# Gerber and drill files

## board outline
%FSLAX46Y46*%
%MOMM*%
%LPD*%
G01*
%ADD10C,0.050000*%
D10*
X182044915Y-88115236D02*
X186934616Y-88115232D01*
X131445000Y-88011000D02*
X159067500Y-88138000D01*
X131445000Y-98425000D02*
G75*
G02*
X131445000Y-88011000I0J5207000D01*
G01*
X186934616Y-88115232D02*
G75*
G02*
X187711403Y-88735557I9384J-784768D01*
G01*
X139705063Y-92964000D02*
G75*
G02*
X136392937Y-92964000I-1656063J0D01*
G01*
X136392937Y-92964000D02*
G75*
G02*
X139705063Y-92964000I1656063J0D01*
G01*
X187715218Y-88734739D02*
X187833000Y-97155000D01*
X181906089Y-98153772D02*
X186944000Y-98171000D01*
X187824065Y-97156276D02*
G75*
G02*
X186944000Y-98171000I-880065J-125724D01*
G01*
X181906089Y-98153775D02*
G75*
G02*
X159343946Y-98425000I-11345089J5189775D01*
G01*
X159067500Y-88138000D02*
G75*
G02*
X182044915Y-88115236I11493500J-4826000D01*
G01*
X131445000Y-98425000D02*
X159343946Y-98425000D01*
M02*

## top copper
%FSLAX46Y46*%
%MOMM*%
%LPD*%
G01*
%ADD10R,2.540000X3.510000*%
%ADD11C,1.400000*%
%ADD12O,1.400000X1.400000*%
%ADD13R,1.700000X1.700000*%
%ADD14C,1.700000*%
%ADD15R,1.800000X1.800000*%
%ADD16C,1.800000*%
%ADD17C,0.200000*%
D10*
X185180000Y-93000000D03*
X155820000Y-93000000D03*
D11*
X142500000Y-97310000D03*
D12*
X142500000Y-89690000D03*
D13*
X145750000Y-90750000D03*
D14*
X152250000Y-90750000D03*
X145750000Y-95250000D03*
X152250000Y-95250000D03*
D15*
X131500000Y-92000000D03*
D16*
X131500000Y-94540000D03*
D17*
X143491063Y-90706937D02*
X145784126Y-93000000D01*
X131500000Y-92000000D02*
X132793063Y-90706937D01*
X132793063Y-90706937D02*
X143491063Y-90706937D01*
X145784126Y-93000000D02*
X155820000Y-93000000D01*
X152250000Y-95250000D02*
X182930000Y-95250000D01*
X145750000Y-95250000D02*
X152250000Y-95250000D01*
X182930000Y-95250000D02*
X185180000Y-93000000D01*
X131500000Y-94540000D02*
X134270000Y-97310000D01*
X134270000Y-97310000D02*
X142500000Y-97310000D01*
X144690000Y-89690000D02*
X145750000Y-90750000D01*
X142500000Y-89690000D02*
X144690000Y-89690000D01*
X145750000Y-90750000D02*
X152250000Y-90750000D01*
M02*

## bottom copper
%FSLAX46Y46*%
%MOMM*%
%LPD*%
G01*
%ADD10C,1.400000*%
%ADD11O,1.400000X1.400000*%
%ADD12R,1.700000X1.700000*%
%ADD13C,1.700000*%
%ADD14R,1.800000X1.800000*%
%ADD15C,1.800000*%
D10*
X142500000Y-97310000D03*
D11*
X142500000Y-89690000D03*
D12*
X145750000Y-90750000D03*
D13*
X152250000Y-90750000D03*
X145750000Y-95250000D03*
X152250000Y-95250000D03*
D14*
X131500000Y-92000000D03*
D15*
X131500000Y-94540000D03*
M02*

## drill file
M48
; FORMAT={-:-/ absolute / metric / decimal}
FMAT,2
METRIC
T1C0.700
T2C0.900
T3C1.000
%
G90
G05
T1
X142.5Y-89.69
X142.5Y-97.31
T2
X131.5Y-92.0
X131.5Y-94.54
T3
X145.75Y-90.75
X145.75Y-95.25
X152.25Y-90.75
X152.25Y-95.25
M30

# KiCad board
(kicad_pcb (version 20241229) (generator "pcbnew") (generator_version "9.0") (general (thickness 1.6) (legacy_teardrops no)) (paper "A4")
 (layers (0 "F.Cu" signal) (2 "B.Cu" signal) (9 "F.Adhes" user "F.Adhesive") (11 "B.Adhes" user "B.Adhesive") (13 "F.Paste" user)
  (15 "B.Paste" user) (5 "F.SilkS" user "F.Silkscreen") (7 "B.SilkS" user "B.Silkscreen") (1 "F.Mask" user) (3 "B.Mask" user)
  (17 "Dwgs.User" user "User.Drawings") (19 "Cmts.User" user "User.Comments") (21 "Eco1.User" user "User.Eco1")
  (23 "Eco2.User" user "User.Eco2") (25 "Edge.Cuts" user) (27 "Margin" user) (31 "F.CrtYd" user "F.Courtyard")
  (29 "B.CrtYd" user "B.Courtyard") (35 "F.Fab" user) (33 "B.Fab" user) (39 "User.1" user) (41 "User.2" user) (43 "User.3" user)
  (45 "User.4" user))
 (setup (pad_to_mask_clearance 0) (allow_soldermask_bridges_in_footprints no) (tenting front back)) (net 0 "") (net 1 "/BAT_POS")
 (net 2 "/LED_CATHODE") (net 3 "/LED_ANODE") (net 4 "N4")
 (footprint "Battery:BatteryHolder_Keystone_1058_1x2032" (layer "F.Cu") (at 170.5 93 180)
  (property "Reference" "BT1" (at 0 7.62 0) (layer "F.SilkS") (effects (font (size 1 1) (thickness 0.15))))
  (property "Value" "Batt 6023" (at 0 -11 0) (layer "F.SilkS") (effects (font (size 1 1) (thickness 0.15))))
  (pad "1" smd rect (at -14.68 0 180) (size 2.54 3.51) (layers "F.Cu" "F.Mask" "F.Paste") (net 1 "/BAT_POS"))
  (pad "2" smd rect (at 14.68 0 180) (size 2.54 3.51) (layers "F.Cu" "F.Mask" "F.Paste") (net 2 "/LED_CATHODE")))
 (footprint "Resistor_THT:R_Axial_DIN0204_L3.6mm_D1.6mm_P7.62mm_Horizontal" (layer "F.Cu") (at 142.5 97.31 90)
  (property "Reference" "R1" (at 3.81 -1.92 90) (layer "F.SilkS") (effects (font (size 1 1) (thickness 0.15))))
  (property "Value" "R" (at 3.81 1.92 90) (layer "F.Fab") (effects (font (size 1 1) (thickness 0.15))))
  (pad "1" thru_hole circle (at 0 0 90) (size 1.4 1.4) (drill 0.7) (layers "*.Cu" "*.Mask") (remove_unused_layers no) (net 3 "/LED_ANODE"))
  (pad "2" thru_hole oval (at 7.62 0 90) (size 1.4 1.4) (drill 0.7) (layers "*.Cu" "*.Mask") (remove_unused_layers no) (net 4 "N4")))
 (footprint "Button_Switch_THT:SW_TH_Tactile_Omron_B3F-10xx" (layer "F.Cu") (at 145.75 90.75)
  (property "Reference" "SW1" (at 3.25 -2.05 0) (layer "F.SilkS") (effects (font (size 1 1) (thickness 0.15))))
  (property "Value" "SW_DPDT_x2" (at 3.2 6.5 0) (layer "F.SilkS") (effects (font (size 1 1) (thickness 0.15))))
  (pad "1" thru_hole rect (at 0 0) (size 1.7 1.7) (drill 1) (layers "*.Cu" "*.Mask") (remove_unused_layers no) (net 4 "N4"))
  (pad "1" thru_hole circle (at 6.5 0) (size 1.7 1.7) (drill 1) (layers "*.Cu" "*.Mask") (remove_unused_layers no) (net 4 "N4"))
  (pad "2" thru_hole circle (at 0 4.5) (size 1.7 1.7) (drill 1) (layers "*.Cu" "*.Mask") (remove_unused_layers no) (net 1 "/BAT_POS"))
  (pad "2" thru_hole circle (at 6.5 4.5) (size 1.7 1.7) (drill 1) (layers "*.Cu" "*.Mask") (remove_unused_layers no) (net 1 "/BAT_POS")))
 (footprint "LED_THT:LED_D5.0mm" (layer "F.Cu") (at 131.5 92 -90)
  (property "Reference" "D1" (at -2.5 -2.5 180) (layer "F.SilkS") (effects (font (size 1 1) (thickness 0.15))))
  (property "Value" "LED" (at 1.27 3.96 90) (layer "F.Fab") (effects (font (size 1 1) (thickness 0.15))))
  (pad "1" thru_hole rect (at 0 0 270) (size 1.8 1.8) (drill 0.9) (layers "*.Cu" "*.Mask") (remove_unused_layers no) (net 2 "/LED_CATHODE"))
  (pad "2" thru_hole circle (at 2.54 0 270) (size 1.8 1.8) (drill 0.9) (layers "*.Cu" "*.Mask") (remove_unused_layers no)
   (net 3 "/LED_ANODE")))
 (gr_line (start 182.044915 88.115236) (end 186.934616 88.115232) (stroke (width 0.05) (type default)) (layer "Edge.Cuts"))
 (gr_line (start 131.445 88.011) (end 159.0675 88.138) (stroke (width 0.05) (type default)) (layer "Edge.Cuts"))
 (gr_arc (start 131.445 98.425) (mid 126.238 93.218) (end 131.445 88.011) (stroke (width 0.05) (type default)) (layer "Edge.Cuts"))
 (gr_arc (start 186.934616 88.115232) (mid 187.433744 88.28673) (end 187.711403 88.735557) (stroke (width 0.05) (type default))
  (layer "Edge.Cuts"))
 (gr_circle (center 138.049 92.964) (end 139.328 94.016) (stroke (width 0.05) (type default)) (fill no) (layer "Edge.Cuts"))
 (gr_line (start 187.715218 88.734739) (end 187.833 97.155) (stroke (width 0.05) (type default)) (layer "Edge.Cuts"))
 (gr_line (start 181.906089 98.153772) (end 186.944 98.171) (stroke (width 0.05) (type default)) (layer "Edge.Cuts"))
 (gr_arc (start 187.824065 97.156276) (mid 187.615599 97.864474) (end 186.944 98.171) (stroke (width 0.05) (type default))
  (layer "Edge.Cuts"))
 (gr_arc (start 181.906089 98.153775) (mid 170.710963 105.438868) (end 159.343946 98.425) (stroke (width 0.05) (type default))
  (layer "Edge.Cuts"))
 (gr_arc (start 159.0675 88.138) (mid 170.54865 80.498421) (end 182.044915 88.115236) (stroke (width 0.05) (type default))
  (layer "Edge.Cuts"))
 (gr_line (start 131.445 98.425) (end 159.343946 98.425) (stroke (width 0.05) (type default)) (layer "Edge.Cuts"))
 (segment (start 143.491063 90.706937) (end 145.784126 93) (width 0.2) (layer "F.Cu") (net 2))
 (segment (start 131.5 92) (end 132.793063 90.706937) (width 0.2) (layer "F.Cu") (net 2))
 (segment (start 132.793063 90.706937) (end 143.491063 90.706937) (width 0.2) (layer "F.Cu") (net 2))
 (segment (start 145.784126 93) (end 155.82 93) (width 0.2) (layer "F.Cu") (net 2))
 (segment (start 152.25 95.25) (end 182.93 95.25) (width 0.2) (layer "F.Cu") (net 1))
 (segment (start 145.75 95.25) (end 152.25 95.25) (width 0.2) (layer "F.Cu") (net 1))
 (segment (start 182.93 95.25) (end 185.18 93) (width 0.2) (layer "F.Cu") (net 1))
 (segment (start 131.5 94.54) (end 134.27 97.31) (width 0.2) (layer "F.Cu") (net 3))
 (segment (start 134.27 97.31) (end 142.5 97.31) (width 0.2) (layer "F.Cu") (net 3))
 (segment (start 144.69 89.69) (end 145.75 90.75) (width 0.2) (layer "F.Cu") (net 4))
 (segment (start 142.5 89.69) (end 144.69 89.69) (width 0.2) (layer "F.Cu") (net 4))
 (segment (start 145.75 90.75) (end 152.25 90.75) (width 0.2) (layer "F.Cu") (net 4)))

